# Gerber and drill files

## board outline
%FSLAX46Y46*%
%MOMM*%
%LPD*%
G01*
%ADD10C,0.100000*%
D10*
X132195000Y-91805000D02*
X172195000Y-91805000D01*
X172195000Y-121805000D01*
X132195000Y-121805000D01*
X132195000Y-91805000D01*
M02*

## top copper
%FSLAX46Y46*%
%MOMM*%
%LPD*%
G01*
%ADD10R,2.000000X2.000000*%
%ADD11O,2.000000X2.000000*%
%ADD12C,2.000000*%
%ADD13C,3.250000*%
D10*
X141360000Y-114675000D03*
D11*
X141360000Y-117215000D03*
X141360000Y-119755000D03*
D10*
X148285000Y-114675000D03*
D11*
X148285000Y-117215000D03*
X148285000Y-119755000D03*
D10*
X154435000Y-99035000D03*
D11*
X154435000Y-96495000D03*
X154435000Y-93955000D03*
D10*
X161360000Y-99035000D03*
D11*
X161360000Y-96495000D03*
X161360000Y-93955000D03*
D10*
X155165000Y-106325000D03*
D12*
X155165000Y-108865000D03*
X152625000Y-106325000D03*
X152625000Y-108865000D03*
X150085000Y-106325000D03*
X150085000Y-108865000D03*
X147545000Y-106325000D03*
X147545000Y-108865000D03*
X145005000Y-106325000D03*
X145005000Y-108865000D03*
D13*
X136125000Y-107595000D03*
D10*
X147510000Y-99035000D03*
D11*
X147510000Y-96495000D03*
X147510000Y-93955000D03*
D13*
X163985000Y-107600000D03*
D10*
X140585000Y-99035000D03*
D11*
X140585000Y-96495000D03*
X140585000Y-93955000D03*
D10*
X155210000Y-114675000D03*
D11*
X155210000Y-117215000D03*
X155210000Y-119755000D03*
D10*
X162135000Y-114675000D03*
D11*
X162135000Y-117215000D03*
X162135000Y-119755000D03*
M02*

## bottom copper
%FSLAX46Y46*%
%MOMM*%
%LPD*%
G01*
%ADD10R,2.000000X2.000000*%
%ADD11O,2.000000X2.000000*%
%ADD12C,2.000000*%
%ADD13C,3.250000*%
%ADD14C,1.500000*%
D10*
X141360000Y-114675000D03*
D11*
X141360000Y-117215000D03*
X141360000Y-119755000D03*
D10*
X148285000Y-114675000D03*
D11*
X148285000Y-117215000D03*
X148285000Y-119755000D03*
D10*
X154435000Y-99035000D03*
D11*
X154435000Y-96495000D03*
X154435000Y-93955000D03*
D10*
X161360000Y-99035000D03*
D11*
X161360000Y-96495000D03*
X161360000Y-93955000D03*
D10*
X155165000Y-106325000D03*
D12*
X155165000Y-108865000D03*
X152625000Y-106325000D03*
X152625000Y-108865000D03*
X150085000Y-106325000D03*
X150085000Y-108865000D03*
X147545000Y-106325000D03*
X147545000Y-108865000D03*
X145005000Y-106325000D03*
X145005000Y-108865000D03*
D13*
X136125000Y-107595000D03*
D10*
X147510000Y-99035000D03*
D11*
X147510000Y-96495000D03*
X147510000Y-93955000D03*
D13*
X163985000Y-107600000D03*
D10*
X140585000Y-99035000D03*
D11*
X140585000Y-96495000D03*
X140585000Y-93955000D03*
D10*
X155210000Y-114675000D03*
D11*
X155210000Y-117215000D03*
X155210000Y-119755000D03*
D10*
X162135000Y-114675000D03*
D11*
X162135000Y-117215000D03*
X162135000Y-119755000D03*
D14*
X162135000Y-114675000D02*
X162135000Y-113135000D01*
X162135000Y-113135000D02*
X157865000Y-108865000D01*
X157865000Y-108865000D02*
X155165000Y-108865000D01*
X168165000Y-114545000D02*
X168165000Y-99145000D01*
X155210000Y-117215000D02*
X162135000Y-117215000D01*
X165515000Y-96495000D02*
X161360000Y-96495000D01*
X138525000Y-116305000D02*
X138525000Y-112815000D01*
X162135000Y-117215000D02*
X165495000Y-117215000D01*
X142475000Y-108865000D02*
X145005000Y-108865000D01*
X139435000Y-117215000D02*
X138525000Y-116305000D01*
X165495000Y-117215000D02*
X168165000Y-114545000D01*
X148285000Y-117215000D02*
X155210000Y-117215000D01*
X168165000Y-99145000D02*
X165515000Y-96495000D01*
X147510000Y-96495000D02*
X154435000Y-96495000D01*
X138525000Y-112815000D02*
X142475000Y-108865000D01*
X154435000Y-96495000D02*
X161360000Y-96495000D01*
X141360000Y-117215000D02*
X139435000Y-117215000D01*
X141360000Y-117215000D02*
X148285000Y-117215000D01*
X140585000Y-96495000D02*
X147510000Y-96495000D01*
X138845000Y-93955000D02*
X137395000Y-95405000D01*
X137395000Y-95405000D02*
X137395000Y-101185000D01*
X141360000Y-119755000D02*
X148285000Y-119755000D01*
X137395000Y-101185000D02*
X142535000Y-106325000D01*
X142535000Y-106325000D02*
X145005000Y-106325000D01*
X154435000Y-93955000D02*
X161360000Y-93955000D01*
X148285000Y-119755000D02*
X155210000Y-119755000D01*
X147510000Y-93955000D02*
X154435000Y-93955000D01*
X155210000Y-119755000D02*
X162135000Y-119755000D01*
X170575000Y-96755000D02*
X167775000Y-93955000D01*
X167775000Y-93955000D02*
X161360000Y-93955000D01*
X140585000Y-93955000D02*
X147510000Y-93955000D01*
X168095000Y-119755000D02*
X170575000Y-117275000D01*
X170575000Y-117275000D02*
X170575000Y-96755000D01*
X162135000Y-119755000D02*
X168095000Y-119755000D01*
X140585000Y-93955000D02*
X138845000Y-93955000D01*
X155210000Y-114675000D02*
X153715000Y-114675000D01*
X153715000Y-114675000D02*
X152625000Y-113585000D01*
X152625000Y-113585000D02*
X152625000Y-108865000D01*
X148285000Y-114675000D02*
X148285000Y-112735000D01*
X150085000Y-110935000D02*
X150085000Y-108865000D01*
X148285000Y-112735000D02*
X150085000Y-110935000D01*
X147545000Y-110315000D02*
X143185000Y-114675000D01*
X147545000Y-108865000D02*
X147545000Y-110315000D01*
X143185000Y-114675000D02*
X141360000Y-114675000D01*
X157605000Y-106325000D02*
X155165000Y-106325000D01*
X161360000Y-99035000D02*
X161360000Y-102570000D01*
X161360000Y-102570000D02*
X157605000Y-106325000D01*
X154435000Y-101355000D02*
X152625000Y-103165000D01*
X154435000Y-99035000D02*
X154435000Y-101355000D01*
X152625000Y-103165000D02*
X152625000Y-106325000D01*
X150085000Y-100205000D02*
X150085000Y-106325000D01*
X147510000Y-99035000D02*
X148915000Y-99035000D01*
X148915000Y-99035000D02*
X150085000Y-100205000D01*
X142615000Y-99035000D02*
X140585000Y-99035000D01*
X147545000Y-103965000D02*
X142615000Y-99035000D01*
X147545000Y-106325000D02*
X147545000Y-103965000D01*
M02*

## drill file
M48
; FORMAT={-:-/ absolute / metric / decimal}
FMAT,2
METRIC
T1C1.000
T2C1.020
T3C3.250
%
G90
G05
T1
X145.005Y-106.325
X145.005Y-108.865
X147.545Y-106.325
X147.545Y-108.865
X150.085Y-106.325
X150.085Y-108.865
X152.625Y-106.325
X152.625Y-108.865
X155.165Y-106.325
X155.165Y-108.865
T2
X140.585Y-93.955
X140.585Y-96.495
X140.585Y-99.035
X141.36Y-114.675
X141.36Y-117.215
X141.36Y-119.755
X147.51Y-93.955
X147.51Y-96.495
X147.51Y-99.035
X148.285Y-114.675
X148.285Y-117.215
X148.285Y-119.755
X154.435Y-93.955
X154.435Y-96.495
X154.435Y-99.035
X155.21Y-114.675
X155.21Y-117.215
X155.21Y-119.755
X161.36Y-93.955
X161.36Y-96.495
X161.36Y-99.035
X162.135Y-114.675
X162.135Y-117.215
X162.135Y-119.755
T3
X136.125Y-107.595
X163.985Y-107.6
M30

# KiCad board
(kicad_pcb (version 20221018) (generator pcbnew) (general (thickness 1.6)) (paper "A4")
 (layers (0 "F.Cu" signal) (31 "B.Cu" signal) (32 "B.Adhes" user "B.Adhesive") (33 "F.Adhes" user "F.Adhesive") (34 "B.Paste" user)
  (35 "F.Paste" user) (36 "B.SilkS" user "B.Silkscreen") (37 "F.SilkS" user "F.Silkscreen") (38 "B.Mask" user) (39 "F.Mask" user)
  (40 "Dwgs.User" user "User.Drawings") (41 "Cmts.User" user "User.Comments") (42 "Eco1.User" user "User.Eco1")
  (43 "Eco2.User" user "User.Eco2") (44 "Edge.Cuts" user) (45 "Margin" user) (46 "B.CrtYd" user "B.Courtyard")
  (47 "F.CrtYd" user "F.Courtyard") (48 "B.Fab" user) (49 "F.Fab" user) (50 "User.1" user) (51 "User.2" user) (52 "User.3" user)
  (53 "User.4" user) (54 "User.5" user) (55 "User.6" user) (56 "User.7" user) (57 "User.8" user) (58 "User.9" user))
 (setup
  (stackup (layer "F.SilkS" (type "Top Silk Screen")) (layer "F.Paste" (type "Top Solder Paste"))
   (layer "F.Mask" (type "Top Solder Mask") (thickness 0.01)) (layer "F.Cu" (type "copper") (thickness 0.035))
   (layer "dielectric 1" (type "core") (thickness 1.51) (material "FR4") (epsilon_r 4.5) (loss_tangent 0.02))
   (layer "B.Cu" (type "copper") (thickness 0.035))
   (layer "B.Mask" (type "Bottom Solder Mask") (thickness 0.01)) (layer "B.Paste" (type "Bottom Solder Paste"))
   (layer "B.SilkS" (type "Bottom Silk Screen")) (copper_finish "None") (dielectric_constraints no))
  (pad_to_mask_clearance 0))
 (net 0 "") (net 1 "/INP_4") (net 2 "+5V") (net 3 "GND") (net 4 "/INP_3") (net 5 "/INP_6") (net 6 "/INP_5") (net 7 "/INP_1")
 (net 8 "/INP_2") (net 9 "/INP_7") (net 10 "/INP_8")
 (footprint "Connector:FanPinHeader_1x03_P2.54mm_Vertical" (layer "F.Cu") (at 141.36 114.675 -90)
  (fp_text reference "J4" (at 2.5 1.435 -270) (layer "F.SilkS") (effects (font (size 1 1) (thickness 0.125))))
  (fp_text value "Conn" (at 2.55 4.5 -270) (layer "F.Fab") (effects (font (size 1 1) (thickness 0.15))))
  (pad "1" thru_hole rect (at 0 0) (size 2 2) (drill 1.02) (layers "*.Cu" "*.Mask") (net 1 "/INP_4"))
  (pad "2" thru_hole oval (at 2.54 0) (size 2 2) (drill 1.02) (layers "*.Cu" "*.Mask") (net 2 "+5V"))
  (pad "3" thru_hole oval (at 5.08 0) (size 2 2) (drill 1.02) (layers "*.Cu" "*.Mask") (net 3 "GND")))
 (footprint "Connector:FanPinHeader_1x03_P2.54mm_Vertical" (layer "F.Cu") (at 148.285 114.675 -90)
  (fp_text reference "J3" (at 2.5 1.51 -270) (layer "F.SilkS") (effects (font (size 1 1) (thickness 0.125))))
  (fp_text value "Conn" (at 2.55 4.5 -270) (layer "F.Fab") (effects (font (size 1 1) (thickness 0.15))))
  (pad "1" thru_hole rect (at 0 0) (size 2 2) (drill 1.02) (layers "*.Cu" "*.Mask") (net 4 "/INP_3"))
  (pad "2" thru_hole oval (at 2.54 0) (size 2 2) (drill 1.02) (layers "*.Cu" "*.Mask") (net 2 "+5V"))
  (pad "3" thru_hole oval (at 5.08 0) (size 2 2) (drill 1.02) (layers "*.Cu" "*.Mask") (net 3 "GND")))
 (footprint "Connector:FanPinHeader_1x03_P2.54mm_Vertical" (layer "F.Cu") (at 154.435 99.035 90)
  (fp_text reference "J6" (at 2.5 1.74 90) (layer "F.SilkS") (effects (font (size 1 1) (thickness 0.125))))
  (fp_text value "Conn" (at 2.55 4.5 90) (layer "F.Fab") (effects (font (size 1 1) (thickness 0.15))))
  (pad "1" thru_hole rect (at 0 0 180) (size 2 2) (drill 1.02) (layers "*.Cu" "*.Mask") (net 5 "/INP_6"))
  (pad "2" thru_hole oval (at 2.54 0 180) (size 2 2) (drill 1.02) (layers "*.Cu" "*.Mask") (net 2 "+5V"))
  (pad "3" thru_hole oval (at 5.08 0 180) (size 2 2) (drill 1.02) (layers "*.Cu" "*.Mask") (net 3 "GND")))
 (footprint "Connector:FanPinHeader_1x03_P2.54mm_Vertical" (layer "F.Cu") (at 161.36 99.035 90)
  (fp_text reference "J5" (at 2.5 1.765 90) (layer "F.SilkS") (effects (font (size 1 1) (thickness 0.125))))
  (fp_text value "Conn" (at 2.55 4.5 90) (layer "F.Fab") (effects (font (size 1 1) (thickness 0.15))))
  (pad "1" thru_hole rect (at 0 0 180) (size 2 2) (drill 1.02) (layers "*.Cu" "*.Mask") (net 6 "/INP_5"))
  (pad "2" thru_hole oval (at 2.54 0 180) (size 2 2) (drill 1.02) (layers "*.Cu" "*.Mask") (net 2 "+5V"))
  (pad "3" thru_hole oval (at 5.08 0 180) (size 2 2) (drill 1.02) (layers "*.Cu" "*.Mask") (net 3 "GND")))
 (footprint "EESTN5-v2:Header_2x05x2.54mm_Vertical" (layer "F.Cu") (at 150.085 107.595 180)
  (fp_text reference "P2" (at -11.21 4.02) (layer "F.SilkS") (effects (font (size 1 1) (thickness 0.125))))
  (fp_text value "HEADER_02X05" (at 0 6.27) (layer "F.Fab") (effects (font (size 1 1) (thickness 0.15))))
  (pad "1" thru_hole rect (at -5.08 1.27 180) (size 2 2) (drill 1) (layers "*.Cu" "*.Mask") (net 6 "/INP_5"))
  (pad "2" thru_hole circle (at -5.08 -1.27 180) (size 2 2) (drill 1) (layers "*.Cu" "*.Mask") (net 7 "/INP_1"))
  (pad "3" thru_hole circle (at -2.54 1.27 180) (size 2 2) (drill 1) (layers "*.Cu" "*.Mask") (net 5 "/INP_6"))
  (pad "4" thru_hole circle (at -2.54 -1.27 180) (size 2 2) (drill 1) (layers "*.Cu" "*.Mask") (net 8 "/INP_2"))
  (pad "5" thru_hole circle (at 0 1.27 180) (size 2 2) (drill 1) (layers "*.Cu" "*.Mask") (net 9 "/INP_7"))
  (pad "6" thru_hole circle (at 0 -1.27 180) (size 2 2) (drill 1) (layers "*.Cu" "*.Mask") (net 4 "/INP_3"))
  (pad "7" thru_hole circle (at 2.54 1.27 180) (size 2 2) (drill 1) (layers "*.Cu" "*.Mask") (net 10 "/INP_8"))
  (pad "8" thru_hole circle (at 2.54 -1.27 180) (size 2 2) (drill 1) (layers "*.Cu" "*.Mask") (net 1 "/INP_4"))
  (pad "9" thru_hole circle (at 5.08 1.27 180) (size 2 2) (drill 1) (layers "*.Cu" "*.Mask") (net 3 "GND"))
  (pad "10" thru_hole circle (at 5.08 -1.27 180) (size 2 2) (drill 1) (layers "*.Cu" "*.Mask") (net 2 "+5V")))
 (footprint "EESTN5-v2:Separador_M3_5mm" (layer "F.Cu") (at 136.125 107.595 90)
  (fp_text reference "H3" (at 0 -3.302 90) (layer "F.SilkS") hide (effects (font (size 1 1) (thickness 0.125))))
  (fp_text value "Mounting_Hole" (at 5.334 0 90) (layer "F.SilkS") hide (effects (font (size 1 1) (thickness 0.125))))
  (pad "1" thru_hole circle (at 0 0 90) (size 3.25 3.25) (drill 3.25) (layers "*.Cu" "F.SilkS")))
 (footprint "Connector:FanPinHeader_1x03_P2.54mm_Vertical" (layer "F.Cu") (at 147.51 99.035 90)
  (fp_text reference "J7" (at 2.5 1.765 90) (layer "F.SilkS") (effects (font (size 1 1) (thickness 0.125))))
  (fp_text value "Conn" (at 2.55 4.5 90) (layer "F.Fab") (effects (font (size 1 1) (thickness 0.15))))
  (pad "1" thru_hole rect (at 0 0 180) (size 2 2) (drill 1.02) (layers "*.Cu" "*.Mask") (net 9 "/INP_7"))
  (pad "2" thru_hole oval (at 2.54 0 180) (size 2 2) (drill 1.02) (layers "*.Cu" "*.Mask") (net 2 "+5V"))
  (pad "3" thru_hole oval (at 5.08 0 180) (size 2 2) (drill 1.02) (layers "*.Cu" "*.Mask") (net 3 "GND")))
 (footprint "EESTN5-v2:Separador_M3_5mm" (layer "F.Cu") (at 163.985 107.6 90)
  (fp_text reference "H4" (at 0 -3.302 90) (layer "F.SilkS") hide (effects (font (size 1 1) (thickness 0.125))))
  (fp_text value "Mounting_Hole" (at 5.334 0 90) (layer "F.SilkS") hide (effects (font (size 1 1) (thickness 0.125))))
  (pad "1" thru_hole circle (at 0 0 90) (size 3.25 3.25) (drill 3.25) (layers "*.Cu" "F.SilkS")))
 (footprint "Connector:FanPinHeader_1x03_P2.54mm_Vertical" (layer "F.Cu") (at 140.585 99.035 90)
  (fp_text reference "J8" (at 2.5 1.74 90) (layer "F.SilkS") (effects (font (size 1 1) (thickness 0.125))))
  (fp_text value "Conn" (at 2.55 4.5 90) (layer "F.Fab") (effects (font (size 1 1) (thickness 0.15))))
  (pad "1" thru_hole rect (at 0 0 180) (size 2 2) (drill 1.02) (layers "*.Cu" "*.Mask") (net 10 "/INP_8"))
  (pad "2" thru_hole oval (at 2.54 0 180) (size 2 2) (drill 1.02) (layers "*.Cu" "*.Mask") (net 2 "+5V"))
  (pad "3" thru_hole oval (at 5.08 0 180) (size 2 2) (drill 1.02) (layers "*.Cu" "*.Mask") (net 3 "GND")))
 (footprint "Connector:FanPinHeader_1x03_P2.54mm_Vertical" (layer "F.Cu") (at 155.21 114.675 -90)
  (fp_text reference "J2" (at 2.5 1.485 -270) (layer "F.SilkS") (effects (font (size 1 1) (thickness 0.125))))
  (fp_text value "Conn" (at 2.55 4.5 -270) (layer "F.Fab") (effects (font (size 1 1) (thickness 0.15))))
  (pad "1" thru_hole rect (at 0 0) (size 2 2) (drill 1.02) (layers "*.Cu" "*.Mask") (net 8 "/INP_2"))
  (pad "2" thru_hole oval (at 2.54 0) (size 2 2) (drill 1.02) (layers "*.Cu" "*.Mask") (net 2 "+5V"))
  (pad "3" thru_hole oval (at 5.08 0) (size 2 2) (drill 1.02) (layers "*.Cu" "*.Mask") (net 3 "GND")))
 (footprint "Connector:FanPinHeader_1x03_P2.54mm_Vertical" (layer "F.Cu") (at 162.135 114.675 -90)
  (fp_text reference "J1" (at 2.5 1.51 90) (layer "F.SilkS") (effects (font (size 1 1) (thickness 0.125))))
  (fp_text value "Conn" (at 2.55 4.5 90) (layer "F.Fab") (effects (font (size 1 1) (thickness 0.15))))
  (pad "1" thru_hole rect (at 0 0) (size 2 2) (drill 1.02) (layers "*.Cu" "*.Mask") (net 7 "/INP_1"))
  (pad "2" thru_hole oval (at 2.54 0) (size 2 2) (drill 1.02) (layers "*.Cu" "*.Mask") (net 2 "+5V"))
  (pad "3" thru_hole oval (at 5.08 0) (size 2 2) (drill 1.02) (layers "*.Cu" "*.Mask") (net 3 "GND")))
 (gr_rect (start 132.195 91.805) (end 172.195 121.805) (stroke (width 0.1) (type default)) (fill none) (layer "Edge.Cuts"))
 (segment (start 162.135 114.675) (end 162.135 113.135) (width 1.5) (layer "B.Cu") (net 7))
 (segment (start 162.135 113.135) (end 157.865 108.865) (width 1.5) (layer "B.Cu") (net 7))
 (segment (start 157.865 108.865) (end 155.165 108.865) (width 1.5) (layer "B.Cu") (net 7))
 (segment (start 168.165 114.545) (end 168.165 99.145) (width 1.5) (layer "B.Cu") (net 2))
 (segment (start 155.21 117.215) (end 162.135 117.215) (width 1.5) (layer "B.Cu") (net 2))
 (segment (start 165.515 96.495) (end 161.36 96.495) (width 1.5) (layer "B.Cu") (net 2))
 (segment (start 138.525 116.305) (end 138.525 112.815) (width 1.5) (layer "B.Cu") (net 2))
 (segment (start 162.135 117.215) (end 165.495 117.215) (width 1.5) (layer "B.Cu") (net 2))
 (segment (start 142.475 108.865) (end 145.005 108.865) (width 1.5) (layer "B.Cu") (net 2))
 (segment (start 139.435 117.215) (end 138.525 116.305) (width 1.5) (layer "B.Cu") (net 2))
 (segment (start 165.495 117.215) (end 168.165 114.545) (width 1.5) (layer "B.Cu") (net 2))
 (segment (start 148.285 117.215) (end 155.21 117.215) (width 1.5) (layer "B.Cu") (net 2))
 (segment (start 168.165 99.145) (end 165.515 96.495) (width 1.5) (layer "B.Cu") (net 2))
 (segment (start 147.51 96.495) (end 154.435 96.495) (width 1.5) (layer "B.Cu") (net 2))
 (segment (start 138.525 112.815) (end 142.475 108.865) (width 1.5) (layer "B.Cu") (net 2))
 (segment (start 154.435 96.495) (end 161.36 96.495) (width 1.5) (layer "B.Cu") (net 2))
 (segment (start 141.36 117.215) (end 139.435 117.215) (width 1.5) (layer "B.Cu") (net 2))
 (segment (start 141.36 117.215) (end 148.285 117.215) (width 1.5) (layer "B.Cu") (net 2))
 (segment (start 140.585 96.495) (end 147.51 96.495) (width 1.5) (layer "B.Cu") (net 2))
 (segment (start 138.845 93.955) (end 137.395 95.405) (width 1.5) (layer "B.Cu") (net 3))
 (segment (start 137.395 95.405) (end 137.395 101.185) (width 1.5) (layer "B.Cu") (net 3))
 (segment (start 141.36 119.755) (end 148.285 119.755) (width 1.5) (layer "B.Cu") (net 3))
 (segment (start 137.395 101.185) (end 142.535 106.325) (width 1.5) (layer "B.Cu") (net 3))
 (segment (start 142.535 106.325) (end 145.005 106.325) (width 1.5) (layer "B.Cu") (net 3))
 (segment (start 154.435 93.955) (end 161.36 93.955) (width 1.5) (layer "B.Cu") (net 3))
 (segment (start 148.285 119.755) (end 155.21 119.755) (width 1.5) (layer "B.Cu") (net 3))
 (segment (start 147.51 93.955) (end 154.435 93.955) (width 1.5) (layer "B.Cu") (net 3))
 (segment (start 155.21 119.755) (end 162.135 119.755) (width 1.5) (layer "B.Cu") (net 3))
 (segment (start 170.575 96.755) (end 167.775 93.955) (width 1.5) (layer "B.Cu") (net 3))
 (segment (start 167.775 93.955) (end 161.36 93.955) (width 1.5) (layer "B.Cu") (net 3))
 (segment (start 140.585 93.955) (end 147.51 93.955) (width 1.5) (layer "B.Cu") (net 3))
 (segment (start 168.095 119.755) (end 170.575 117.275) (width 1.5) (layer "B.Cu") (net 3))
 (segment (start 170.575 117.275) (end 170.575 96.755) (width 1.5) (layer "B.Cu") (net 3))
 (segment (start 162.135 119.755) (end 168.095 119.755) (width 1.5) (layer "B.Cu") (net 3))
 (segment (start 140.585 93.955) (end 138.845 93.955) (width 1.5) (layer "B.Cu") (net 3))
 (segment (start 155.21 114.675) (end 153.715 114.675) (width 1.5) (layer "B.Cu") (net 8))
 (segment (start 153.715 114.675) (end 152.625 113.585) (width 1.5) (layer "B.Cu") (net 8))
 (segment (start 152.625 113.585) (end 152.625 108.865) (width 1.5) (layer "B.Cu") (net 8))
 (segment (start 148.285 114.675) (end 148.285 112.735) (width 1.5) (layer "B.Cu") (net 4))
 (segment (start 150.085 110.935) (end 150.085 108.865) (width 1.5) (layer "B.Cu") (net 4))
 (segment (start 148.285 112.735) (end 150.085 110.935) (width 1.5) (layer "B.Cu") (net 4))
 (segment (start 147.545 110.315) (end 143.185 114.675) (width 1.5) (layer "B.Cu") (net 1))
 (segment (start 147.545 108.865) (end 147.545 110.315) (width 1.5) (layer "B.Cu") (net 1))
 (segment (start 143.185 114.675) (end 141.36 114.675) (width 1.5) (layer "B.Cu") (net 1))
 (segment (start 157.605 106.325) (end 155.165 106.325) (width 1.5) (layer "B.Cu") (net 6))
 (segment (start 161.36 99.035) (end 161.36 102.57) (width 1.5) (layer "B.Cu") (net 6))
 (segment (start 161.36 102.57) (end 157.605 106.325) (width 1.5) (layer "B.Cu") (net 6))
 (segment (start 154.435 101.355) (end 152.625 103.165) (width 1.5) (layer "B.Cu") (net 5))
 (segment (start 154.435 99.035) (end 154.435 101.355) (width 1.5) (layer "B.Cu") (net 5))
 (segment (start 152.625 103.165) (end 152.625 106.325) (width 1.5) (layer "B.Cu") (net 5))
 (segment (start 150.085 100.205) (end 150.085 106.325) (width 1.5) (layer "B.Cu") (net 9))
 (segment (start 147.51 99.035) (end 148.915 99.035) (width 1.5) (layer "B.Cu") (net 9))
 (segment (start 148.915 99.035) (end 150.085 100.205) (width 1.5) (layer "B.Cu") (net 9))
 (segment (start 142.615 99.035) (end 140.585 99.035) (width 1.5) (layer "B.Cu") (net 10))
 (segment (start 147.545 103.965) (end 142.615 99.035) (width 1.5) (layer "B.Cu") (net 10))
 (segment (start 147.545 106.325) (end 147.545 103.965) (width 1.5) (layer "B.Cu") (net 10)))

